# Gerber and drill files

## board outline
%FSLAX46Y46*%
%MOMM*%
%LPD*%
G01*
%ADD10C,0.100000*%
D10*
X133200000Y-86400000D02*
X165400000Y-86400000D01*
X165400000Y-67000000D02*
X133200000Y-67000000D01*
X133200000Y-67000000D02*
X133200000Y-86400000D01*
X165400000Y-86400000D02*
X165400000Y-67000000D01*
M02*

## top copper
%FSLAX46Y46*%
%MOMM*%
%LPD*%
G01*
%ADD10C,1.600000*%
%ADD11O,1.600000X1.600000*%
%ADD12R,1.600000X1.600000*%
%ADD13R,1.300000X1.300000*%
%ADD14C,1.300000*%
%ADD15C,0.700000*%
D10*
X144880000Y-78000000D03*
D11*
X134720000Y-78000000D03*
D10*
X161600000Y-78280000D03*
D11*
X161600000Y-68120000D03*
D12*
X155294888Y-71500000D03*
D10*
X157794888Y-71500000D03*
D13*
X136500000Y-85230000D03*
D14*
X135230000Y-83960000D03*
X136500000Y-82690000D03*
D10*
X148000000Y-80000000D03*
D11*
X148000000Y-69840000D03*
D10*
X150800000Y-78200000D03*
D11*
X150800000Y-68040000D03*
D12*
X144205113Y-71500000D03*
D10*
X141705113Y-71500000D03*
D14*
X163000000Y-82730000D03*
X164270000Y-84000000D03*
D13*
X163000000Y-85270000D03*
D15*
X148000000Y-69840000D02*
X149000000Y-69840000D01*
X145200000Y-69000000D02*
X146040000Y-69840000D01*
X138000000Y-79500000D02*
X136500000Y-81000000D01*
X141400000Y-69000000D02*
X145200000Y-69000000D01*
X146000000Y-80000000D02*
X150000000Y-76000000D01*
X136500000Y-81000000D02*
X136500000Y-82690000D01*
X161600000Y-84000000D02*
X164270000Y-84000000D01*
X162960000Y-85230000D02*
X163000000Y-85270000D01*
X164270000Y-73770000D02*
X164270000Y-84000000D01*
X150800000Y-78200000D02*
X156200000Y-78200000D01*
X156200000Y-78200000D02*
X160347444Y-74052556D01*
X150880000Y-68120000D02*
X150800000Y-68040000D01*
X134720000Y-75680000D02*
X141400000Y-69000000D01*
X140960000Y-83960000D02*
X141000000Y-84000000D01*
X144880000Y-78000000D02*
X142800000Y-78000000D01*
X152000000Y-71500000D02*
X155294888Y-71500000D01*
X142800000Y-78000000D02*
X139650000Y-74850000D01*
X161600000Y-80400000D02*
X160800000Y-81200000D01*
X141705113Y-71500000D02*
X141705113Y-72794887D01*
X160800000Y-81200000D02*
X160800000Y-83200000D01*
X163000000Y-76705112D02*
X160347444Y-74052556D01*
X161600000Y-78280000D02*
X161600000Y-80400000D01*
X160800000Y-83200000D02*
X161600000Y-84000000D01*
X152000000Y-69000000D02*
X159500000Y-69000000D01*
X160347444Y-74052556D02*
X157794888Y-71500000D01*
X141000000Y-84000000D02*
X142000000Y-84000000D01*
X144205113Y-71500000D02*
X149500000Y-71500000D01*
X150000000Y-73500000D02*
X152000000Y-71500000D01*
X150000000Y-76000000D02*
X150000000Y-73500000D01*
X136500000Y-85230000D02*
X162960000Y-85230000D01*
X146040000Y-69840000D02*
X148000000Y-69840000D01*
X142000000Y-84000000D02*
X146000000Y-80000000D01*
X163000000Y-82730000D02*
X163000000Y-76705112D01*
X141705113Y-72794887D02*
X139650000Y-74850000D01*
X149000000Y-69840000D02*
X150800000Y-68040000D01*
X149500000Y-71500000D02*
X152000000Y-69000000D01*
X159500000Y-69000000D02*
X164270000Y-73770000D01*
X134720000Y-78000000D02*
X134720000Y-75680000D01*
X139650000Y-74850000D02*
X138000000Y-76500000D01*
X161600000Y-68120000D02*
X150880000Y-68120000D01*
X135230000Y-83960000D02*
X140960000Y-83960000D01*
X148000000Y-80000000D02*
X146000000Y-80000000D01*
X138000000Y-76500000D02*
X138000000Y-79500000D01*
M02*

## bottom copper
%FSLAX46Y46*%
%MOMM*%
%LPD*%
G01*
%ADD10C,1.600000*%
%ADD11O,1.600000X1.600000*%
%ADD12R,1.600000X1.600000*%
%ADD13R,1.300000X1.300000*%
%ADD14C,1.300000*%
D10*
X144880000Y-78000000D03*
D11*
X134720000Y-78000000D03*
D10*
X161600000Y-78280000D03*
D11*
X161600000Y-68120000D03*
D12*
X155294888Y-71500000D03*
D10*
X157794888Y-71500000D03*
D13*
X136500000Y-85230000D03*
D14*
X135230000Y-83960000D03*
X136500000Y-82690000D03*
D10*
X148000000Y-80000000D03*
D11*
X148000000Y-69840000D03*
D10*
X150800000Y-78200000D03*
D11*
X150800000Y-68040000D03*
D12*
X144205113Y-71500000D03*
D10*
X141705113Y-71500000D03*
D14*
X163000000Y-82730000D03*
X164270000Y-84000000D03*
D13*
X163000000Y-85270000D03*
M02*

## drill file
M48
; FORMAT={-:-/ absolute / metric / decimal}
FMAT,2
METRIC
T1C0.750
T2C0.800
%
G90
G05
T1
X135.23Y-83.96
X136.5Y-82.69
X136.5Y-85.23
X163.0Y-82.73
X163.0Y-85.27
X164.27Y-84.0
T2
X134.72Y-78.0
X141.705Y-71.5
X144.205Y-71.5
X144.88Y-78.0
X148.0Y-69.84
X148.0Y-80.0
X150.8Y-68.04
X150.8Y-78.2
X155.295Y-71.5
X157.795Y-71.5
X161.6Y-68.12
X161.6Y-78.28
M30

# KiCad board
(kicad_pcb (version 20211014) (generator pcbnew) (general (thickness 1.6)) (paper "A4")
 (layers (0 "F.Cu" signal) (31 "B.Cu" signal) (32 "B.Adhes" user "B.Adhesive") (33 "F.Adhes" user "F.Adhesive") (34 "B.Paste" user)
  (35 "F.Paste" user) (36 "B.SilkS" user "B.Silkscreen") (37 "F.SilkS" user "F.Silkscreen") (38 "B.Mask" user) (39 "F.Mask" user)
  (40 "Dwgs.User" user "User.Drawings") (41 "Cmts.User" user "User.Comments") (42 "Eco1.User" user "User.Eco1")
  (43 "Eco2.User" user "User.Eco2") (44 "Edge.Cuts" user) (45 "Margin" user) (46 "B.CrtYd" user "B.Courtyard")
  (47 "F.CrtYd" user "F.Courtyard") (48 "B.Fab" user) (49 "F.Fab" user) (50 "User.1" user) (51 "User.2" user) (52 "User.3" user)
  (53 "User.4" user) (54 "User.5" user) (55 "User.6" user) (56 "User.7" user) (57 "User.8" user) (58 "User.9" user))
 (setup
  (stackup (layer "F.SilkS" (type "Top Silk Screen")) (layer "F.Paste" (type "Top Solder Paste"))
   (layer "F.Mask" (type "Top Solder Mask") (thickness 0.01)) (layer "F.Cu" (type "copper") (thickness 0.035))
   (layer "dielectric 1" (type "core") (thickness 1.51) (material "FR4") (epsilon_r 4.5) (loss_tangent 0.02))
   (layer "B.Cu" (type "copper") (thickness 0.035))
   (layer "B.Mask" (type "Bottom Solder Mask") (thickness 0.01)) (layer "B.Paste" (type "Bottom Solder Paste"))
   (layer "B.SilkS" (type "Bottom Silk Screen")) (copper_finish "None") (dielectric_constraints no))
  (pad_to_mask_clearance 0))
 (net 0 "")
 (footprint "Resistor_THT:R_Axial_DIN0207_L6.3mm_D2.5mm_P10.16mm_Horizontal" (layer "F.Cu") (at 144.88 78 180)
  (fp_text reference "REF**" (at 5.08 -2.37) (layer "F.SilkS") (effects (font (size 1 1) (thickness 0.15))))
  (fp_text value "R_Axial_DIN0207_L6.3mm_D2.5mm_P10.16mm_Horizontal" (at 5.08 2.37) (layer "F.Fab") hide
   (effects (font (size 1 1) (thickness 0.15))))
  (pad "1" thru_hole circle (at 0 0 180) (size 1.6 1.6) (drill 0.8) (layers *.Cu *.Mask))
  (pad "2" thru_hole oval (at 10.16 0 180) (size 1.6 1.6) (drill 0.8) (layers *.Cu *.Mask)))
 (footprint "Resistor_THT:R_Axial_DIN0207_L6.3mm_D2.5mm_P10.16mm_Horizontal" (layer "F.Cu") (at 161.6 78.28 90)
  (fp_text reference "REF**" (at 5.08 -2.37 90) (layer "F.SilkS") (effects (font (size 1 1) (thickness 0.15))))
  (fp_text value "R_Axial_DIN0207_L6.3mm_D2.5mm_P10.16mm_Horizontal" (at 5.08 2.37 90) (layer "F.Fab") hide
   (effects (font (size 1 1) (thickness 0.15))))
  (pad "1" thru_hole circle (at 0 0 90) (size 1.6 1.6) (drill 0.8) (layers *.Cu *.Mask))
  (pad "2" thru_hole oval (at 10.16 0 90) (size 1.6 1.6) (drill 0.8) (layers *.Cu *.Mask)))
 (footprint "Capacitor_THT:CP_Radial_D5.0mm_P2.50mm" (layer "F.Cu") (at 155.294888 71.5)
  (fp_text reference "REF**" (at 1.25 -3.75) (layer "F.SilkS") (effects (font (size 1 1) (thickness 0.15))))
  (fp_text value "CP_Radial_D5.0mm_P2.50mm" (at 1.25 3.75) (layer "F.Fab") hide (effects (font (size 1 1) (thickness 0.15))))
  (pad "1" thru_hole rect (at 0 0) (size 1.6 1.6) (drill 0.8) (layers *.Cu *.Mask))
  (pad "2" thru_hole circle (at 2.5 0) (size 1.6 1.6) (drill 0.8) (layers *.Cu *.Mask)))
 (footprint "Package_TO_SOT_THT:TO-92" (layer "F.Cu") (at 136.5 85.23 90)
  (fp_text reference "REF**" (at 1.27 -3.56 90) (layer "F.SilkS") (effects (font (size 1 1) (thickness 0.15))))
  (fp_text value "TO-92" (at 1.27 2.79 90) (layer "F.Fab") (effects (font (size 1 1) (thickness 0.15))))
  (pad "1" thru_hole rect (at 0 0 90) (size 1.3 1.3) (drill 0.75) (layers *.Cu *.Mask))
  (pad "2" thru_hole circle (at 1.27 -1.27 90) (size 1.3 1.3) (drill 0.75) (layers *.Cu *.Mask))
  (pad "3" thru_hole circle (at 2.54 0 90) (size 1.3 1.3) (drill 0.75) (layers *.Cu *.Mask)))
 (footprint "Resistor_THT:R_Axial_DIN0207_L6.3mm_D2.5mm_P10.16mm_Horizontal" (layer "F.Cu") (at 148 80 90)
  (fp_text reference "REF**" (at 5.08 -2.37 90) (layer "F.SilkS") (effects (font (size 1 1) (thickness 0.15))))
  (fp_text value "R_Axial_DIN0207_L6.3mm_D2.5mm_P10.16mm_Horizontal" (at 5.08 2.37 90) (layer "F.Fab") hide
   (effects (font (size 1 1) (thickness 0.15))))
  (pad "1" thru_hole circle (at 0 0 90) (size 1.6 1.6) (drill 0.8) (layers *.Cu *.Mask))
  (pad "2" thru_hole oval (at 10.16 0 90) (size 1.6 1.6) (drill 0.8) (layers *.Cu *.Mask)))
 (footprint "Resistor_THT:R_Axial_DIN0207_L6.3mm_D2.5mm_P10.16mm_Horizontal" (layer "F.Cu") (at 150.8 78.2 90)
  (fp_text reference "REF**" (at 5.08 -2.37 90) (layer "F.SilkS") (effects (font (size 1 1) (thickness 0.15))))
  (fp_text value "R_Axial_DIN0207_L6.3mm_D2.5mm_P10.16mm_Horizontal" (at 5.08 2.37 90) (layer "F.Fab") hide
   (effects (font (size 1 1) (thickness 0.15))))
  (pad "1" thru_hole circle (at 0 0 90) (size 1.6 1.6) (drill 0.8) (layers *.Cu *.Mask))
  (pad "2" thru_hole oval (at 10.16 0 90) (size 1.6 1.6) (drill 0.8) (layers *.Cu *.Mask)))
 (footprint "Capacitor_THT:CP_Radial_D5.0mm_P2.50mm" (layer "F.Cu") (at 144.205113 71.5 180)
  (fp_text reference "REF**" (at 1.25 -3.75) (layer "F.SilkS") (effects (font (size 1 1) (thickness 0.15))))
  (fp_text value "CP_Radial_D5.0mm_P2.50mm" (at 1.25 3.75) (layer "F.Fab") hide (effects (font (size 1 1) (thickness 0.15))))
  (pad "1" thru_hole rect (at 0 0 180) (size 1.6 1.6) (drill 0.8) (layers *.Cu *.Mask))
  (pad "2" thru_hole circle (at 2.5 0 180) (size 1.6 1.6) (drill 0.8) (layers *.Cu *.Mask)))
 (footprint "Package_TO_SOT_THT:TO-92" (layer "F.Cu") (at 163 82.73 -90)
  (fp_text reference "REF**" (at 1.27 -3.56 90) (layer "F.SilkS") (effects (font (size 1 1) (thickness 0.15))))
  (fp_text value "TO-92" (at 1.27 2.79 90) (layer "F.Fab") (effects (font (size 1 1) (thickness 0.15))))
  (pad "1" thru_hole circle (at 0 0 270) (size 1.3 1.3) (drill 0.75) (layers *.Cu *.Mask))
  (pad "2" thru_hole circle (at 1.27 -1.27 270) (size 1.3 1.3) (drill 0.75) (layers *.Cu *.Mask))
  (pad "3" thru_hole rect (at 2.54 0 270) (size 1.3 1.3) (drill 0.75) (layers *.Cu *.Mask)))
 (gr_line (start 133.2 86.4) (end 165.4 86.4) (layer "Edge.Cuts") (width 0.1))
 (gr_line (start 165.4 67) (end 133.2 67) (layer "Edge.Cuts") (width 0.1))
 (gr_line (start 133.2 67) (end 133.2 86.4) (layer "Edge.Cuts") (width 0.1))
 (gr_line (start 165.4 86.4) (end 165.4 67) (layer "Edge.Cuts") (width 0.1))
 (segment (start 148 69.84) (end 149 69.84) (width 0.7) (layer "F.Cu") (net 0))
 (segment (start 145.2 69) (end 146.04 69.84) (width 0.7) (layer "F.Cu") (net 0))
 (segment (start 138 79.5) (end 136.5 81) (width 0.7) (layer "F.Cu") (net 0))
 (segment (start 141.4 69) (end 145.2 69) (width 0.7) (layer "F.Cu") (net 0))
 (segment (start 146 80) (end 150 76) (width 0.7) (layer "F.Cu") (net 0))
 (segment (start 136.5 81) (end 136.5 82.69) (width 0.7) (layer "F.Cu") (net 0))
 (segment (start 161.6 84) (end 164.27 84) (width 0.7) (layer "F.Cu") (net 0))
 (segment (start 162.96 85.23) (end 163 85.27) (width 0.7) (layer "F.Cu") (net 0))
 (segment (start 164.27 73.77) (end 164.27 84) (width 0.7) (layer "F.Cu") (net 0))
 (segment (start 150.8 78.2) (end 156.2 78.2) (width 0.7) (layer "F.Cu") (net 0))
 (segment (start 156.2 78.2) (end 160.347444 74.052556) (width 0.7) (layer "F.Cu") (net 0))
 (segment (start 150.88 68.12) (end 150.8 68.04) (width 0.7) (layer "F.Cu") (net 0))
 (segment (start 134.72 75.68) (end 141.4 69) (width 0.7) (layer "F.Cu") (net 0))
 (segment (start 140.96 83.96) (end 141 84) (width 0.7) (layer "F.Cu") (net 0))
 (segment (start 144.88 78) (end 142.8 78) (width 0.7) (layer "F.Cu") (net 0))
 (segment (start 152 71.5) (end 155.294888 71.5) (width 0.7) (layer "F.Cu") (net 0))
 (segment (start 142.8 78) (end 139.65 74.85) (width 0.7) (layer "F.Cu") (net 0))
 (segment (start 161.6 80.4) (end 160.8 81.2) (width 0.7) (layer "F.Cu") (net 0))
 (segment (start 141.705113 71.5) (end 141.705113 72.794887) (width 0.7) (layer "F.Cu") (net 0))
 (segment (start 160.8 81.2) (end 160.8 83.2) (width 0.7) (layer "F.Cu") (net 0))
 (segment (start 163 76.705112) (end 160.347444 74.052556) (width 0.7) (layer "F.Cu") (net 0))
 (segment (start 161.6 78.28) (end 161.6 80.4) (width 0.7) (layer "F.Cu") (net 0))
 (segment (start 160.8 83.2) (end 161.6 84) (width 0.7) (layer "F.Cu") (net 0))
 (segment (start 152 69) (end 159.5 69) (width 0.7) (layer "F.Cu") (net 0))
 (segment (start 160.347444 74.052556) (end 157.794888 71.5) (width 0.7) (layer "F.Cu") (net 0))
 (segment (start 141 84) (end 142 84) (width 0.7) (layer "F.Cu") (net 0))
 (segment (start 144.205113 71.5) (end 149.5 71.5) (width 0.7) (layer "F.Cu") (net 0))
 (segment (start 150 73.5) (end 152 71.5) (width 0.7) (layer "F.Cu") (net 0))
 (segment (start 150 76) (end 150 73.5) (width 0.7) (layer "F.Cu") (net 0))
 (segment (start 136.5 85.23) (end 162.96 85.23) (width 0.7) (layer "F.Cu") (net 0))
 (segment (start 146.04 69.84) (end 148 69.84) (width 0.7) (layer "F.Cu") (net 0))
 (segment (start 142 84) (end 146 80) (width 0.7) (layer "F.Cu") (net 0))
 (segment (start 163 82.73) (end 163 76.705112) (width 0.7) (layer "F.Cu") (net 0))
 (segment (start 141.705113 72.794887) (end 139.65 74.85) (width 0.7) (layer "F.Cu") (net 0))
 (segment (start 149 69.84) (end 150.8 68.04) (width 0.7) (layer "F.Cu") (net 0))
 (segment (start 149.5 71.5) (end 152 69) (width 0.7) (layer "F.Cu") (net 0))
 (segment (start 159.5 69) (end 164.27 73.77) (width 0.7) (layer "F.Cu") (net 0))
 (segment (start 134.72 78) (end 134.72 75.68) (width 0.7) (layer "F.Cu") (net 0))
 (segment (start 139.65 74.85) (end 138 76.5) (width 0.7) (layer "F.Cu") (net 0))
 (segment (start 161.6 68.12) (end 150.88 68.12) (width 0.7) (layer "F.Cu") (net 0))
 (segment (start 135.23 83.96) (end 140.96 83.96) (width 0.7) (layer "F.Cu") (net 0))
 (segment (start 148 80) (end 146 80) (width 0.7) (layer "F.Cu") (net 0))
 (segment (start 138 76.5) (end 138 79.5) (width 0.7) (layer "F.Cu") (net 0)))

